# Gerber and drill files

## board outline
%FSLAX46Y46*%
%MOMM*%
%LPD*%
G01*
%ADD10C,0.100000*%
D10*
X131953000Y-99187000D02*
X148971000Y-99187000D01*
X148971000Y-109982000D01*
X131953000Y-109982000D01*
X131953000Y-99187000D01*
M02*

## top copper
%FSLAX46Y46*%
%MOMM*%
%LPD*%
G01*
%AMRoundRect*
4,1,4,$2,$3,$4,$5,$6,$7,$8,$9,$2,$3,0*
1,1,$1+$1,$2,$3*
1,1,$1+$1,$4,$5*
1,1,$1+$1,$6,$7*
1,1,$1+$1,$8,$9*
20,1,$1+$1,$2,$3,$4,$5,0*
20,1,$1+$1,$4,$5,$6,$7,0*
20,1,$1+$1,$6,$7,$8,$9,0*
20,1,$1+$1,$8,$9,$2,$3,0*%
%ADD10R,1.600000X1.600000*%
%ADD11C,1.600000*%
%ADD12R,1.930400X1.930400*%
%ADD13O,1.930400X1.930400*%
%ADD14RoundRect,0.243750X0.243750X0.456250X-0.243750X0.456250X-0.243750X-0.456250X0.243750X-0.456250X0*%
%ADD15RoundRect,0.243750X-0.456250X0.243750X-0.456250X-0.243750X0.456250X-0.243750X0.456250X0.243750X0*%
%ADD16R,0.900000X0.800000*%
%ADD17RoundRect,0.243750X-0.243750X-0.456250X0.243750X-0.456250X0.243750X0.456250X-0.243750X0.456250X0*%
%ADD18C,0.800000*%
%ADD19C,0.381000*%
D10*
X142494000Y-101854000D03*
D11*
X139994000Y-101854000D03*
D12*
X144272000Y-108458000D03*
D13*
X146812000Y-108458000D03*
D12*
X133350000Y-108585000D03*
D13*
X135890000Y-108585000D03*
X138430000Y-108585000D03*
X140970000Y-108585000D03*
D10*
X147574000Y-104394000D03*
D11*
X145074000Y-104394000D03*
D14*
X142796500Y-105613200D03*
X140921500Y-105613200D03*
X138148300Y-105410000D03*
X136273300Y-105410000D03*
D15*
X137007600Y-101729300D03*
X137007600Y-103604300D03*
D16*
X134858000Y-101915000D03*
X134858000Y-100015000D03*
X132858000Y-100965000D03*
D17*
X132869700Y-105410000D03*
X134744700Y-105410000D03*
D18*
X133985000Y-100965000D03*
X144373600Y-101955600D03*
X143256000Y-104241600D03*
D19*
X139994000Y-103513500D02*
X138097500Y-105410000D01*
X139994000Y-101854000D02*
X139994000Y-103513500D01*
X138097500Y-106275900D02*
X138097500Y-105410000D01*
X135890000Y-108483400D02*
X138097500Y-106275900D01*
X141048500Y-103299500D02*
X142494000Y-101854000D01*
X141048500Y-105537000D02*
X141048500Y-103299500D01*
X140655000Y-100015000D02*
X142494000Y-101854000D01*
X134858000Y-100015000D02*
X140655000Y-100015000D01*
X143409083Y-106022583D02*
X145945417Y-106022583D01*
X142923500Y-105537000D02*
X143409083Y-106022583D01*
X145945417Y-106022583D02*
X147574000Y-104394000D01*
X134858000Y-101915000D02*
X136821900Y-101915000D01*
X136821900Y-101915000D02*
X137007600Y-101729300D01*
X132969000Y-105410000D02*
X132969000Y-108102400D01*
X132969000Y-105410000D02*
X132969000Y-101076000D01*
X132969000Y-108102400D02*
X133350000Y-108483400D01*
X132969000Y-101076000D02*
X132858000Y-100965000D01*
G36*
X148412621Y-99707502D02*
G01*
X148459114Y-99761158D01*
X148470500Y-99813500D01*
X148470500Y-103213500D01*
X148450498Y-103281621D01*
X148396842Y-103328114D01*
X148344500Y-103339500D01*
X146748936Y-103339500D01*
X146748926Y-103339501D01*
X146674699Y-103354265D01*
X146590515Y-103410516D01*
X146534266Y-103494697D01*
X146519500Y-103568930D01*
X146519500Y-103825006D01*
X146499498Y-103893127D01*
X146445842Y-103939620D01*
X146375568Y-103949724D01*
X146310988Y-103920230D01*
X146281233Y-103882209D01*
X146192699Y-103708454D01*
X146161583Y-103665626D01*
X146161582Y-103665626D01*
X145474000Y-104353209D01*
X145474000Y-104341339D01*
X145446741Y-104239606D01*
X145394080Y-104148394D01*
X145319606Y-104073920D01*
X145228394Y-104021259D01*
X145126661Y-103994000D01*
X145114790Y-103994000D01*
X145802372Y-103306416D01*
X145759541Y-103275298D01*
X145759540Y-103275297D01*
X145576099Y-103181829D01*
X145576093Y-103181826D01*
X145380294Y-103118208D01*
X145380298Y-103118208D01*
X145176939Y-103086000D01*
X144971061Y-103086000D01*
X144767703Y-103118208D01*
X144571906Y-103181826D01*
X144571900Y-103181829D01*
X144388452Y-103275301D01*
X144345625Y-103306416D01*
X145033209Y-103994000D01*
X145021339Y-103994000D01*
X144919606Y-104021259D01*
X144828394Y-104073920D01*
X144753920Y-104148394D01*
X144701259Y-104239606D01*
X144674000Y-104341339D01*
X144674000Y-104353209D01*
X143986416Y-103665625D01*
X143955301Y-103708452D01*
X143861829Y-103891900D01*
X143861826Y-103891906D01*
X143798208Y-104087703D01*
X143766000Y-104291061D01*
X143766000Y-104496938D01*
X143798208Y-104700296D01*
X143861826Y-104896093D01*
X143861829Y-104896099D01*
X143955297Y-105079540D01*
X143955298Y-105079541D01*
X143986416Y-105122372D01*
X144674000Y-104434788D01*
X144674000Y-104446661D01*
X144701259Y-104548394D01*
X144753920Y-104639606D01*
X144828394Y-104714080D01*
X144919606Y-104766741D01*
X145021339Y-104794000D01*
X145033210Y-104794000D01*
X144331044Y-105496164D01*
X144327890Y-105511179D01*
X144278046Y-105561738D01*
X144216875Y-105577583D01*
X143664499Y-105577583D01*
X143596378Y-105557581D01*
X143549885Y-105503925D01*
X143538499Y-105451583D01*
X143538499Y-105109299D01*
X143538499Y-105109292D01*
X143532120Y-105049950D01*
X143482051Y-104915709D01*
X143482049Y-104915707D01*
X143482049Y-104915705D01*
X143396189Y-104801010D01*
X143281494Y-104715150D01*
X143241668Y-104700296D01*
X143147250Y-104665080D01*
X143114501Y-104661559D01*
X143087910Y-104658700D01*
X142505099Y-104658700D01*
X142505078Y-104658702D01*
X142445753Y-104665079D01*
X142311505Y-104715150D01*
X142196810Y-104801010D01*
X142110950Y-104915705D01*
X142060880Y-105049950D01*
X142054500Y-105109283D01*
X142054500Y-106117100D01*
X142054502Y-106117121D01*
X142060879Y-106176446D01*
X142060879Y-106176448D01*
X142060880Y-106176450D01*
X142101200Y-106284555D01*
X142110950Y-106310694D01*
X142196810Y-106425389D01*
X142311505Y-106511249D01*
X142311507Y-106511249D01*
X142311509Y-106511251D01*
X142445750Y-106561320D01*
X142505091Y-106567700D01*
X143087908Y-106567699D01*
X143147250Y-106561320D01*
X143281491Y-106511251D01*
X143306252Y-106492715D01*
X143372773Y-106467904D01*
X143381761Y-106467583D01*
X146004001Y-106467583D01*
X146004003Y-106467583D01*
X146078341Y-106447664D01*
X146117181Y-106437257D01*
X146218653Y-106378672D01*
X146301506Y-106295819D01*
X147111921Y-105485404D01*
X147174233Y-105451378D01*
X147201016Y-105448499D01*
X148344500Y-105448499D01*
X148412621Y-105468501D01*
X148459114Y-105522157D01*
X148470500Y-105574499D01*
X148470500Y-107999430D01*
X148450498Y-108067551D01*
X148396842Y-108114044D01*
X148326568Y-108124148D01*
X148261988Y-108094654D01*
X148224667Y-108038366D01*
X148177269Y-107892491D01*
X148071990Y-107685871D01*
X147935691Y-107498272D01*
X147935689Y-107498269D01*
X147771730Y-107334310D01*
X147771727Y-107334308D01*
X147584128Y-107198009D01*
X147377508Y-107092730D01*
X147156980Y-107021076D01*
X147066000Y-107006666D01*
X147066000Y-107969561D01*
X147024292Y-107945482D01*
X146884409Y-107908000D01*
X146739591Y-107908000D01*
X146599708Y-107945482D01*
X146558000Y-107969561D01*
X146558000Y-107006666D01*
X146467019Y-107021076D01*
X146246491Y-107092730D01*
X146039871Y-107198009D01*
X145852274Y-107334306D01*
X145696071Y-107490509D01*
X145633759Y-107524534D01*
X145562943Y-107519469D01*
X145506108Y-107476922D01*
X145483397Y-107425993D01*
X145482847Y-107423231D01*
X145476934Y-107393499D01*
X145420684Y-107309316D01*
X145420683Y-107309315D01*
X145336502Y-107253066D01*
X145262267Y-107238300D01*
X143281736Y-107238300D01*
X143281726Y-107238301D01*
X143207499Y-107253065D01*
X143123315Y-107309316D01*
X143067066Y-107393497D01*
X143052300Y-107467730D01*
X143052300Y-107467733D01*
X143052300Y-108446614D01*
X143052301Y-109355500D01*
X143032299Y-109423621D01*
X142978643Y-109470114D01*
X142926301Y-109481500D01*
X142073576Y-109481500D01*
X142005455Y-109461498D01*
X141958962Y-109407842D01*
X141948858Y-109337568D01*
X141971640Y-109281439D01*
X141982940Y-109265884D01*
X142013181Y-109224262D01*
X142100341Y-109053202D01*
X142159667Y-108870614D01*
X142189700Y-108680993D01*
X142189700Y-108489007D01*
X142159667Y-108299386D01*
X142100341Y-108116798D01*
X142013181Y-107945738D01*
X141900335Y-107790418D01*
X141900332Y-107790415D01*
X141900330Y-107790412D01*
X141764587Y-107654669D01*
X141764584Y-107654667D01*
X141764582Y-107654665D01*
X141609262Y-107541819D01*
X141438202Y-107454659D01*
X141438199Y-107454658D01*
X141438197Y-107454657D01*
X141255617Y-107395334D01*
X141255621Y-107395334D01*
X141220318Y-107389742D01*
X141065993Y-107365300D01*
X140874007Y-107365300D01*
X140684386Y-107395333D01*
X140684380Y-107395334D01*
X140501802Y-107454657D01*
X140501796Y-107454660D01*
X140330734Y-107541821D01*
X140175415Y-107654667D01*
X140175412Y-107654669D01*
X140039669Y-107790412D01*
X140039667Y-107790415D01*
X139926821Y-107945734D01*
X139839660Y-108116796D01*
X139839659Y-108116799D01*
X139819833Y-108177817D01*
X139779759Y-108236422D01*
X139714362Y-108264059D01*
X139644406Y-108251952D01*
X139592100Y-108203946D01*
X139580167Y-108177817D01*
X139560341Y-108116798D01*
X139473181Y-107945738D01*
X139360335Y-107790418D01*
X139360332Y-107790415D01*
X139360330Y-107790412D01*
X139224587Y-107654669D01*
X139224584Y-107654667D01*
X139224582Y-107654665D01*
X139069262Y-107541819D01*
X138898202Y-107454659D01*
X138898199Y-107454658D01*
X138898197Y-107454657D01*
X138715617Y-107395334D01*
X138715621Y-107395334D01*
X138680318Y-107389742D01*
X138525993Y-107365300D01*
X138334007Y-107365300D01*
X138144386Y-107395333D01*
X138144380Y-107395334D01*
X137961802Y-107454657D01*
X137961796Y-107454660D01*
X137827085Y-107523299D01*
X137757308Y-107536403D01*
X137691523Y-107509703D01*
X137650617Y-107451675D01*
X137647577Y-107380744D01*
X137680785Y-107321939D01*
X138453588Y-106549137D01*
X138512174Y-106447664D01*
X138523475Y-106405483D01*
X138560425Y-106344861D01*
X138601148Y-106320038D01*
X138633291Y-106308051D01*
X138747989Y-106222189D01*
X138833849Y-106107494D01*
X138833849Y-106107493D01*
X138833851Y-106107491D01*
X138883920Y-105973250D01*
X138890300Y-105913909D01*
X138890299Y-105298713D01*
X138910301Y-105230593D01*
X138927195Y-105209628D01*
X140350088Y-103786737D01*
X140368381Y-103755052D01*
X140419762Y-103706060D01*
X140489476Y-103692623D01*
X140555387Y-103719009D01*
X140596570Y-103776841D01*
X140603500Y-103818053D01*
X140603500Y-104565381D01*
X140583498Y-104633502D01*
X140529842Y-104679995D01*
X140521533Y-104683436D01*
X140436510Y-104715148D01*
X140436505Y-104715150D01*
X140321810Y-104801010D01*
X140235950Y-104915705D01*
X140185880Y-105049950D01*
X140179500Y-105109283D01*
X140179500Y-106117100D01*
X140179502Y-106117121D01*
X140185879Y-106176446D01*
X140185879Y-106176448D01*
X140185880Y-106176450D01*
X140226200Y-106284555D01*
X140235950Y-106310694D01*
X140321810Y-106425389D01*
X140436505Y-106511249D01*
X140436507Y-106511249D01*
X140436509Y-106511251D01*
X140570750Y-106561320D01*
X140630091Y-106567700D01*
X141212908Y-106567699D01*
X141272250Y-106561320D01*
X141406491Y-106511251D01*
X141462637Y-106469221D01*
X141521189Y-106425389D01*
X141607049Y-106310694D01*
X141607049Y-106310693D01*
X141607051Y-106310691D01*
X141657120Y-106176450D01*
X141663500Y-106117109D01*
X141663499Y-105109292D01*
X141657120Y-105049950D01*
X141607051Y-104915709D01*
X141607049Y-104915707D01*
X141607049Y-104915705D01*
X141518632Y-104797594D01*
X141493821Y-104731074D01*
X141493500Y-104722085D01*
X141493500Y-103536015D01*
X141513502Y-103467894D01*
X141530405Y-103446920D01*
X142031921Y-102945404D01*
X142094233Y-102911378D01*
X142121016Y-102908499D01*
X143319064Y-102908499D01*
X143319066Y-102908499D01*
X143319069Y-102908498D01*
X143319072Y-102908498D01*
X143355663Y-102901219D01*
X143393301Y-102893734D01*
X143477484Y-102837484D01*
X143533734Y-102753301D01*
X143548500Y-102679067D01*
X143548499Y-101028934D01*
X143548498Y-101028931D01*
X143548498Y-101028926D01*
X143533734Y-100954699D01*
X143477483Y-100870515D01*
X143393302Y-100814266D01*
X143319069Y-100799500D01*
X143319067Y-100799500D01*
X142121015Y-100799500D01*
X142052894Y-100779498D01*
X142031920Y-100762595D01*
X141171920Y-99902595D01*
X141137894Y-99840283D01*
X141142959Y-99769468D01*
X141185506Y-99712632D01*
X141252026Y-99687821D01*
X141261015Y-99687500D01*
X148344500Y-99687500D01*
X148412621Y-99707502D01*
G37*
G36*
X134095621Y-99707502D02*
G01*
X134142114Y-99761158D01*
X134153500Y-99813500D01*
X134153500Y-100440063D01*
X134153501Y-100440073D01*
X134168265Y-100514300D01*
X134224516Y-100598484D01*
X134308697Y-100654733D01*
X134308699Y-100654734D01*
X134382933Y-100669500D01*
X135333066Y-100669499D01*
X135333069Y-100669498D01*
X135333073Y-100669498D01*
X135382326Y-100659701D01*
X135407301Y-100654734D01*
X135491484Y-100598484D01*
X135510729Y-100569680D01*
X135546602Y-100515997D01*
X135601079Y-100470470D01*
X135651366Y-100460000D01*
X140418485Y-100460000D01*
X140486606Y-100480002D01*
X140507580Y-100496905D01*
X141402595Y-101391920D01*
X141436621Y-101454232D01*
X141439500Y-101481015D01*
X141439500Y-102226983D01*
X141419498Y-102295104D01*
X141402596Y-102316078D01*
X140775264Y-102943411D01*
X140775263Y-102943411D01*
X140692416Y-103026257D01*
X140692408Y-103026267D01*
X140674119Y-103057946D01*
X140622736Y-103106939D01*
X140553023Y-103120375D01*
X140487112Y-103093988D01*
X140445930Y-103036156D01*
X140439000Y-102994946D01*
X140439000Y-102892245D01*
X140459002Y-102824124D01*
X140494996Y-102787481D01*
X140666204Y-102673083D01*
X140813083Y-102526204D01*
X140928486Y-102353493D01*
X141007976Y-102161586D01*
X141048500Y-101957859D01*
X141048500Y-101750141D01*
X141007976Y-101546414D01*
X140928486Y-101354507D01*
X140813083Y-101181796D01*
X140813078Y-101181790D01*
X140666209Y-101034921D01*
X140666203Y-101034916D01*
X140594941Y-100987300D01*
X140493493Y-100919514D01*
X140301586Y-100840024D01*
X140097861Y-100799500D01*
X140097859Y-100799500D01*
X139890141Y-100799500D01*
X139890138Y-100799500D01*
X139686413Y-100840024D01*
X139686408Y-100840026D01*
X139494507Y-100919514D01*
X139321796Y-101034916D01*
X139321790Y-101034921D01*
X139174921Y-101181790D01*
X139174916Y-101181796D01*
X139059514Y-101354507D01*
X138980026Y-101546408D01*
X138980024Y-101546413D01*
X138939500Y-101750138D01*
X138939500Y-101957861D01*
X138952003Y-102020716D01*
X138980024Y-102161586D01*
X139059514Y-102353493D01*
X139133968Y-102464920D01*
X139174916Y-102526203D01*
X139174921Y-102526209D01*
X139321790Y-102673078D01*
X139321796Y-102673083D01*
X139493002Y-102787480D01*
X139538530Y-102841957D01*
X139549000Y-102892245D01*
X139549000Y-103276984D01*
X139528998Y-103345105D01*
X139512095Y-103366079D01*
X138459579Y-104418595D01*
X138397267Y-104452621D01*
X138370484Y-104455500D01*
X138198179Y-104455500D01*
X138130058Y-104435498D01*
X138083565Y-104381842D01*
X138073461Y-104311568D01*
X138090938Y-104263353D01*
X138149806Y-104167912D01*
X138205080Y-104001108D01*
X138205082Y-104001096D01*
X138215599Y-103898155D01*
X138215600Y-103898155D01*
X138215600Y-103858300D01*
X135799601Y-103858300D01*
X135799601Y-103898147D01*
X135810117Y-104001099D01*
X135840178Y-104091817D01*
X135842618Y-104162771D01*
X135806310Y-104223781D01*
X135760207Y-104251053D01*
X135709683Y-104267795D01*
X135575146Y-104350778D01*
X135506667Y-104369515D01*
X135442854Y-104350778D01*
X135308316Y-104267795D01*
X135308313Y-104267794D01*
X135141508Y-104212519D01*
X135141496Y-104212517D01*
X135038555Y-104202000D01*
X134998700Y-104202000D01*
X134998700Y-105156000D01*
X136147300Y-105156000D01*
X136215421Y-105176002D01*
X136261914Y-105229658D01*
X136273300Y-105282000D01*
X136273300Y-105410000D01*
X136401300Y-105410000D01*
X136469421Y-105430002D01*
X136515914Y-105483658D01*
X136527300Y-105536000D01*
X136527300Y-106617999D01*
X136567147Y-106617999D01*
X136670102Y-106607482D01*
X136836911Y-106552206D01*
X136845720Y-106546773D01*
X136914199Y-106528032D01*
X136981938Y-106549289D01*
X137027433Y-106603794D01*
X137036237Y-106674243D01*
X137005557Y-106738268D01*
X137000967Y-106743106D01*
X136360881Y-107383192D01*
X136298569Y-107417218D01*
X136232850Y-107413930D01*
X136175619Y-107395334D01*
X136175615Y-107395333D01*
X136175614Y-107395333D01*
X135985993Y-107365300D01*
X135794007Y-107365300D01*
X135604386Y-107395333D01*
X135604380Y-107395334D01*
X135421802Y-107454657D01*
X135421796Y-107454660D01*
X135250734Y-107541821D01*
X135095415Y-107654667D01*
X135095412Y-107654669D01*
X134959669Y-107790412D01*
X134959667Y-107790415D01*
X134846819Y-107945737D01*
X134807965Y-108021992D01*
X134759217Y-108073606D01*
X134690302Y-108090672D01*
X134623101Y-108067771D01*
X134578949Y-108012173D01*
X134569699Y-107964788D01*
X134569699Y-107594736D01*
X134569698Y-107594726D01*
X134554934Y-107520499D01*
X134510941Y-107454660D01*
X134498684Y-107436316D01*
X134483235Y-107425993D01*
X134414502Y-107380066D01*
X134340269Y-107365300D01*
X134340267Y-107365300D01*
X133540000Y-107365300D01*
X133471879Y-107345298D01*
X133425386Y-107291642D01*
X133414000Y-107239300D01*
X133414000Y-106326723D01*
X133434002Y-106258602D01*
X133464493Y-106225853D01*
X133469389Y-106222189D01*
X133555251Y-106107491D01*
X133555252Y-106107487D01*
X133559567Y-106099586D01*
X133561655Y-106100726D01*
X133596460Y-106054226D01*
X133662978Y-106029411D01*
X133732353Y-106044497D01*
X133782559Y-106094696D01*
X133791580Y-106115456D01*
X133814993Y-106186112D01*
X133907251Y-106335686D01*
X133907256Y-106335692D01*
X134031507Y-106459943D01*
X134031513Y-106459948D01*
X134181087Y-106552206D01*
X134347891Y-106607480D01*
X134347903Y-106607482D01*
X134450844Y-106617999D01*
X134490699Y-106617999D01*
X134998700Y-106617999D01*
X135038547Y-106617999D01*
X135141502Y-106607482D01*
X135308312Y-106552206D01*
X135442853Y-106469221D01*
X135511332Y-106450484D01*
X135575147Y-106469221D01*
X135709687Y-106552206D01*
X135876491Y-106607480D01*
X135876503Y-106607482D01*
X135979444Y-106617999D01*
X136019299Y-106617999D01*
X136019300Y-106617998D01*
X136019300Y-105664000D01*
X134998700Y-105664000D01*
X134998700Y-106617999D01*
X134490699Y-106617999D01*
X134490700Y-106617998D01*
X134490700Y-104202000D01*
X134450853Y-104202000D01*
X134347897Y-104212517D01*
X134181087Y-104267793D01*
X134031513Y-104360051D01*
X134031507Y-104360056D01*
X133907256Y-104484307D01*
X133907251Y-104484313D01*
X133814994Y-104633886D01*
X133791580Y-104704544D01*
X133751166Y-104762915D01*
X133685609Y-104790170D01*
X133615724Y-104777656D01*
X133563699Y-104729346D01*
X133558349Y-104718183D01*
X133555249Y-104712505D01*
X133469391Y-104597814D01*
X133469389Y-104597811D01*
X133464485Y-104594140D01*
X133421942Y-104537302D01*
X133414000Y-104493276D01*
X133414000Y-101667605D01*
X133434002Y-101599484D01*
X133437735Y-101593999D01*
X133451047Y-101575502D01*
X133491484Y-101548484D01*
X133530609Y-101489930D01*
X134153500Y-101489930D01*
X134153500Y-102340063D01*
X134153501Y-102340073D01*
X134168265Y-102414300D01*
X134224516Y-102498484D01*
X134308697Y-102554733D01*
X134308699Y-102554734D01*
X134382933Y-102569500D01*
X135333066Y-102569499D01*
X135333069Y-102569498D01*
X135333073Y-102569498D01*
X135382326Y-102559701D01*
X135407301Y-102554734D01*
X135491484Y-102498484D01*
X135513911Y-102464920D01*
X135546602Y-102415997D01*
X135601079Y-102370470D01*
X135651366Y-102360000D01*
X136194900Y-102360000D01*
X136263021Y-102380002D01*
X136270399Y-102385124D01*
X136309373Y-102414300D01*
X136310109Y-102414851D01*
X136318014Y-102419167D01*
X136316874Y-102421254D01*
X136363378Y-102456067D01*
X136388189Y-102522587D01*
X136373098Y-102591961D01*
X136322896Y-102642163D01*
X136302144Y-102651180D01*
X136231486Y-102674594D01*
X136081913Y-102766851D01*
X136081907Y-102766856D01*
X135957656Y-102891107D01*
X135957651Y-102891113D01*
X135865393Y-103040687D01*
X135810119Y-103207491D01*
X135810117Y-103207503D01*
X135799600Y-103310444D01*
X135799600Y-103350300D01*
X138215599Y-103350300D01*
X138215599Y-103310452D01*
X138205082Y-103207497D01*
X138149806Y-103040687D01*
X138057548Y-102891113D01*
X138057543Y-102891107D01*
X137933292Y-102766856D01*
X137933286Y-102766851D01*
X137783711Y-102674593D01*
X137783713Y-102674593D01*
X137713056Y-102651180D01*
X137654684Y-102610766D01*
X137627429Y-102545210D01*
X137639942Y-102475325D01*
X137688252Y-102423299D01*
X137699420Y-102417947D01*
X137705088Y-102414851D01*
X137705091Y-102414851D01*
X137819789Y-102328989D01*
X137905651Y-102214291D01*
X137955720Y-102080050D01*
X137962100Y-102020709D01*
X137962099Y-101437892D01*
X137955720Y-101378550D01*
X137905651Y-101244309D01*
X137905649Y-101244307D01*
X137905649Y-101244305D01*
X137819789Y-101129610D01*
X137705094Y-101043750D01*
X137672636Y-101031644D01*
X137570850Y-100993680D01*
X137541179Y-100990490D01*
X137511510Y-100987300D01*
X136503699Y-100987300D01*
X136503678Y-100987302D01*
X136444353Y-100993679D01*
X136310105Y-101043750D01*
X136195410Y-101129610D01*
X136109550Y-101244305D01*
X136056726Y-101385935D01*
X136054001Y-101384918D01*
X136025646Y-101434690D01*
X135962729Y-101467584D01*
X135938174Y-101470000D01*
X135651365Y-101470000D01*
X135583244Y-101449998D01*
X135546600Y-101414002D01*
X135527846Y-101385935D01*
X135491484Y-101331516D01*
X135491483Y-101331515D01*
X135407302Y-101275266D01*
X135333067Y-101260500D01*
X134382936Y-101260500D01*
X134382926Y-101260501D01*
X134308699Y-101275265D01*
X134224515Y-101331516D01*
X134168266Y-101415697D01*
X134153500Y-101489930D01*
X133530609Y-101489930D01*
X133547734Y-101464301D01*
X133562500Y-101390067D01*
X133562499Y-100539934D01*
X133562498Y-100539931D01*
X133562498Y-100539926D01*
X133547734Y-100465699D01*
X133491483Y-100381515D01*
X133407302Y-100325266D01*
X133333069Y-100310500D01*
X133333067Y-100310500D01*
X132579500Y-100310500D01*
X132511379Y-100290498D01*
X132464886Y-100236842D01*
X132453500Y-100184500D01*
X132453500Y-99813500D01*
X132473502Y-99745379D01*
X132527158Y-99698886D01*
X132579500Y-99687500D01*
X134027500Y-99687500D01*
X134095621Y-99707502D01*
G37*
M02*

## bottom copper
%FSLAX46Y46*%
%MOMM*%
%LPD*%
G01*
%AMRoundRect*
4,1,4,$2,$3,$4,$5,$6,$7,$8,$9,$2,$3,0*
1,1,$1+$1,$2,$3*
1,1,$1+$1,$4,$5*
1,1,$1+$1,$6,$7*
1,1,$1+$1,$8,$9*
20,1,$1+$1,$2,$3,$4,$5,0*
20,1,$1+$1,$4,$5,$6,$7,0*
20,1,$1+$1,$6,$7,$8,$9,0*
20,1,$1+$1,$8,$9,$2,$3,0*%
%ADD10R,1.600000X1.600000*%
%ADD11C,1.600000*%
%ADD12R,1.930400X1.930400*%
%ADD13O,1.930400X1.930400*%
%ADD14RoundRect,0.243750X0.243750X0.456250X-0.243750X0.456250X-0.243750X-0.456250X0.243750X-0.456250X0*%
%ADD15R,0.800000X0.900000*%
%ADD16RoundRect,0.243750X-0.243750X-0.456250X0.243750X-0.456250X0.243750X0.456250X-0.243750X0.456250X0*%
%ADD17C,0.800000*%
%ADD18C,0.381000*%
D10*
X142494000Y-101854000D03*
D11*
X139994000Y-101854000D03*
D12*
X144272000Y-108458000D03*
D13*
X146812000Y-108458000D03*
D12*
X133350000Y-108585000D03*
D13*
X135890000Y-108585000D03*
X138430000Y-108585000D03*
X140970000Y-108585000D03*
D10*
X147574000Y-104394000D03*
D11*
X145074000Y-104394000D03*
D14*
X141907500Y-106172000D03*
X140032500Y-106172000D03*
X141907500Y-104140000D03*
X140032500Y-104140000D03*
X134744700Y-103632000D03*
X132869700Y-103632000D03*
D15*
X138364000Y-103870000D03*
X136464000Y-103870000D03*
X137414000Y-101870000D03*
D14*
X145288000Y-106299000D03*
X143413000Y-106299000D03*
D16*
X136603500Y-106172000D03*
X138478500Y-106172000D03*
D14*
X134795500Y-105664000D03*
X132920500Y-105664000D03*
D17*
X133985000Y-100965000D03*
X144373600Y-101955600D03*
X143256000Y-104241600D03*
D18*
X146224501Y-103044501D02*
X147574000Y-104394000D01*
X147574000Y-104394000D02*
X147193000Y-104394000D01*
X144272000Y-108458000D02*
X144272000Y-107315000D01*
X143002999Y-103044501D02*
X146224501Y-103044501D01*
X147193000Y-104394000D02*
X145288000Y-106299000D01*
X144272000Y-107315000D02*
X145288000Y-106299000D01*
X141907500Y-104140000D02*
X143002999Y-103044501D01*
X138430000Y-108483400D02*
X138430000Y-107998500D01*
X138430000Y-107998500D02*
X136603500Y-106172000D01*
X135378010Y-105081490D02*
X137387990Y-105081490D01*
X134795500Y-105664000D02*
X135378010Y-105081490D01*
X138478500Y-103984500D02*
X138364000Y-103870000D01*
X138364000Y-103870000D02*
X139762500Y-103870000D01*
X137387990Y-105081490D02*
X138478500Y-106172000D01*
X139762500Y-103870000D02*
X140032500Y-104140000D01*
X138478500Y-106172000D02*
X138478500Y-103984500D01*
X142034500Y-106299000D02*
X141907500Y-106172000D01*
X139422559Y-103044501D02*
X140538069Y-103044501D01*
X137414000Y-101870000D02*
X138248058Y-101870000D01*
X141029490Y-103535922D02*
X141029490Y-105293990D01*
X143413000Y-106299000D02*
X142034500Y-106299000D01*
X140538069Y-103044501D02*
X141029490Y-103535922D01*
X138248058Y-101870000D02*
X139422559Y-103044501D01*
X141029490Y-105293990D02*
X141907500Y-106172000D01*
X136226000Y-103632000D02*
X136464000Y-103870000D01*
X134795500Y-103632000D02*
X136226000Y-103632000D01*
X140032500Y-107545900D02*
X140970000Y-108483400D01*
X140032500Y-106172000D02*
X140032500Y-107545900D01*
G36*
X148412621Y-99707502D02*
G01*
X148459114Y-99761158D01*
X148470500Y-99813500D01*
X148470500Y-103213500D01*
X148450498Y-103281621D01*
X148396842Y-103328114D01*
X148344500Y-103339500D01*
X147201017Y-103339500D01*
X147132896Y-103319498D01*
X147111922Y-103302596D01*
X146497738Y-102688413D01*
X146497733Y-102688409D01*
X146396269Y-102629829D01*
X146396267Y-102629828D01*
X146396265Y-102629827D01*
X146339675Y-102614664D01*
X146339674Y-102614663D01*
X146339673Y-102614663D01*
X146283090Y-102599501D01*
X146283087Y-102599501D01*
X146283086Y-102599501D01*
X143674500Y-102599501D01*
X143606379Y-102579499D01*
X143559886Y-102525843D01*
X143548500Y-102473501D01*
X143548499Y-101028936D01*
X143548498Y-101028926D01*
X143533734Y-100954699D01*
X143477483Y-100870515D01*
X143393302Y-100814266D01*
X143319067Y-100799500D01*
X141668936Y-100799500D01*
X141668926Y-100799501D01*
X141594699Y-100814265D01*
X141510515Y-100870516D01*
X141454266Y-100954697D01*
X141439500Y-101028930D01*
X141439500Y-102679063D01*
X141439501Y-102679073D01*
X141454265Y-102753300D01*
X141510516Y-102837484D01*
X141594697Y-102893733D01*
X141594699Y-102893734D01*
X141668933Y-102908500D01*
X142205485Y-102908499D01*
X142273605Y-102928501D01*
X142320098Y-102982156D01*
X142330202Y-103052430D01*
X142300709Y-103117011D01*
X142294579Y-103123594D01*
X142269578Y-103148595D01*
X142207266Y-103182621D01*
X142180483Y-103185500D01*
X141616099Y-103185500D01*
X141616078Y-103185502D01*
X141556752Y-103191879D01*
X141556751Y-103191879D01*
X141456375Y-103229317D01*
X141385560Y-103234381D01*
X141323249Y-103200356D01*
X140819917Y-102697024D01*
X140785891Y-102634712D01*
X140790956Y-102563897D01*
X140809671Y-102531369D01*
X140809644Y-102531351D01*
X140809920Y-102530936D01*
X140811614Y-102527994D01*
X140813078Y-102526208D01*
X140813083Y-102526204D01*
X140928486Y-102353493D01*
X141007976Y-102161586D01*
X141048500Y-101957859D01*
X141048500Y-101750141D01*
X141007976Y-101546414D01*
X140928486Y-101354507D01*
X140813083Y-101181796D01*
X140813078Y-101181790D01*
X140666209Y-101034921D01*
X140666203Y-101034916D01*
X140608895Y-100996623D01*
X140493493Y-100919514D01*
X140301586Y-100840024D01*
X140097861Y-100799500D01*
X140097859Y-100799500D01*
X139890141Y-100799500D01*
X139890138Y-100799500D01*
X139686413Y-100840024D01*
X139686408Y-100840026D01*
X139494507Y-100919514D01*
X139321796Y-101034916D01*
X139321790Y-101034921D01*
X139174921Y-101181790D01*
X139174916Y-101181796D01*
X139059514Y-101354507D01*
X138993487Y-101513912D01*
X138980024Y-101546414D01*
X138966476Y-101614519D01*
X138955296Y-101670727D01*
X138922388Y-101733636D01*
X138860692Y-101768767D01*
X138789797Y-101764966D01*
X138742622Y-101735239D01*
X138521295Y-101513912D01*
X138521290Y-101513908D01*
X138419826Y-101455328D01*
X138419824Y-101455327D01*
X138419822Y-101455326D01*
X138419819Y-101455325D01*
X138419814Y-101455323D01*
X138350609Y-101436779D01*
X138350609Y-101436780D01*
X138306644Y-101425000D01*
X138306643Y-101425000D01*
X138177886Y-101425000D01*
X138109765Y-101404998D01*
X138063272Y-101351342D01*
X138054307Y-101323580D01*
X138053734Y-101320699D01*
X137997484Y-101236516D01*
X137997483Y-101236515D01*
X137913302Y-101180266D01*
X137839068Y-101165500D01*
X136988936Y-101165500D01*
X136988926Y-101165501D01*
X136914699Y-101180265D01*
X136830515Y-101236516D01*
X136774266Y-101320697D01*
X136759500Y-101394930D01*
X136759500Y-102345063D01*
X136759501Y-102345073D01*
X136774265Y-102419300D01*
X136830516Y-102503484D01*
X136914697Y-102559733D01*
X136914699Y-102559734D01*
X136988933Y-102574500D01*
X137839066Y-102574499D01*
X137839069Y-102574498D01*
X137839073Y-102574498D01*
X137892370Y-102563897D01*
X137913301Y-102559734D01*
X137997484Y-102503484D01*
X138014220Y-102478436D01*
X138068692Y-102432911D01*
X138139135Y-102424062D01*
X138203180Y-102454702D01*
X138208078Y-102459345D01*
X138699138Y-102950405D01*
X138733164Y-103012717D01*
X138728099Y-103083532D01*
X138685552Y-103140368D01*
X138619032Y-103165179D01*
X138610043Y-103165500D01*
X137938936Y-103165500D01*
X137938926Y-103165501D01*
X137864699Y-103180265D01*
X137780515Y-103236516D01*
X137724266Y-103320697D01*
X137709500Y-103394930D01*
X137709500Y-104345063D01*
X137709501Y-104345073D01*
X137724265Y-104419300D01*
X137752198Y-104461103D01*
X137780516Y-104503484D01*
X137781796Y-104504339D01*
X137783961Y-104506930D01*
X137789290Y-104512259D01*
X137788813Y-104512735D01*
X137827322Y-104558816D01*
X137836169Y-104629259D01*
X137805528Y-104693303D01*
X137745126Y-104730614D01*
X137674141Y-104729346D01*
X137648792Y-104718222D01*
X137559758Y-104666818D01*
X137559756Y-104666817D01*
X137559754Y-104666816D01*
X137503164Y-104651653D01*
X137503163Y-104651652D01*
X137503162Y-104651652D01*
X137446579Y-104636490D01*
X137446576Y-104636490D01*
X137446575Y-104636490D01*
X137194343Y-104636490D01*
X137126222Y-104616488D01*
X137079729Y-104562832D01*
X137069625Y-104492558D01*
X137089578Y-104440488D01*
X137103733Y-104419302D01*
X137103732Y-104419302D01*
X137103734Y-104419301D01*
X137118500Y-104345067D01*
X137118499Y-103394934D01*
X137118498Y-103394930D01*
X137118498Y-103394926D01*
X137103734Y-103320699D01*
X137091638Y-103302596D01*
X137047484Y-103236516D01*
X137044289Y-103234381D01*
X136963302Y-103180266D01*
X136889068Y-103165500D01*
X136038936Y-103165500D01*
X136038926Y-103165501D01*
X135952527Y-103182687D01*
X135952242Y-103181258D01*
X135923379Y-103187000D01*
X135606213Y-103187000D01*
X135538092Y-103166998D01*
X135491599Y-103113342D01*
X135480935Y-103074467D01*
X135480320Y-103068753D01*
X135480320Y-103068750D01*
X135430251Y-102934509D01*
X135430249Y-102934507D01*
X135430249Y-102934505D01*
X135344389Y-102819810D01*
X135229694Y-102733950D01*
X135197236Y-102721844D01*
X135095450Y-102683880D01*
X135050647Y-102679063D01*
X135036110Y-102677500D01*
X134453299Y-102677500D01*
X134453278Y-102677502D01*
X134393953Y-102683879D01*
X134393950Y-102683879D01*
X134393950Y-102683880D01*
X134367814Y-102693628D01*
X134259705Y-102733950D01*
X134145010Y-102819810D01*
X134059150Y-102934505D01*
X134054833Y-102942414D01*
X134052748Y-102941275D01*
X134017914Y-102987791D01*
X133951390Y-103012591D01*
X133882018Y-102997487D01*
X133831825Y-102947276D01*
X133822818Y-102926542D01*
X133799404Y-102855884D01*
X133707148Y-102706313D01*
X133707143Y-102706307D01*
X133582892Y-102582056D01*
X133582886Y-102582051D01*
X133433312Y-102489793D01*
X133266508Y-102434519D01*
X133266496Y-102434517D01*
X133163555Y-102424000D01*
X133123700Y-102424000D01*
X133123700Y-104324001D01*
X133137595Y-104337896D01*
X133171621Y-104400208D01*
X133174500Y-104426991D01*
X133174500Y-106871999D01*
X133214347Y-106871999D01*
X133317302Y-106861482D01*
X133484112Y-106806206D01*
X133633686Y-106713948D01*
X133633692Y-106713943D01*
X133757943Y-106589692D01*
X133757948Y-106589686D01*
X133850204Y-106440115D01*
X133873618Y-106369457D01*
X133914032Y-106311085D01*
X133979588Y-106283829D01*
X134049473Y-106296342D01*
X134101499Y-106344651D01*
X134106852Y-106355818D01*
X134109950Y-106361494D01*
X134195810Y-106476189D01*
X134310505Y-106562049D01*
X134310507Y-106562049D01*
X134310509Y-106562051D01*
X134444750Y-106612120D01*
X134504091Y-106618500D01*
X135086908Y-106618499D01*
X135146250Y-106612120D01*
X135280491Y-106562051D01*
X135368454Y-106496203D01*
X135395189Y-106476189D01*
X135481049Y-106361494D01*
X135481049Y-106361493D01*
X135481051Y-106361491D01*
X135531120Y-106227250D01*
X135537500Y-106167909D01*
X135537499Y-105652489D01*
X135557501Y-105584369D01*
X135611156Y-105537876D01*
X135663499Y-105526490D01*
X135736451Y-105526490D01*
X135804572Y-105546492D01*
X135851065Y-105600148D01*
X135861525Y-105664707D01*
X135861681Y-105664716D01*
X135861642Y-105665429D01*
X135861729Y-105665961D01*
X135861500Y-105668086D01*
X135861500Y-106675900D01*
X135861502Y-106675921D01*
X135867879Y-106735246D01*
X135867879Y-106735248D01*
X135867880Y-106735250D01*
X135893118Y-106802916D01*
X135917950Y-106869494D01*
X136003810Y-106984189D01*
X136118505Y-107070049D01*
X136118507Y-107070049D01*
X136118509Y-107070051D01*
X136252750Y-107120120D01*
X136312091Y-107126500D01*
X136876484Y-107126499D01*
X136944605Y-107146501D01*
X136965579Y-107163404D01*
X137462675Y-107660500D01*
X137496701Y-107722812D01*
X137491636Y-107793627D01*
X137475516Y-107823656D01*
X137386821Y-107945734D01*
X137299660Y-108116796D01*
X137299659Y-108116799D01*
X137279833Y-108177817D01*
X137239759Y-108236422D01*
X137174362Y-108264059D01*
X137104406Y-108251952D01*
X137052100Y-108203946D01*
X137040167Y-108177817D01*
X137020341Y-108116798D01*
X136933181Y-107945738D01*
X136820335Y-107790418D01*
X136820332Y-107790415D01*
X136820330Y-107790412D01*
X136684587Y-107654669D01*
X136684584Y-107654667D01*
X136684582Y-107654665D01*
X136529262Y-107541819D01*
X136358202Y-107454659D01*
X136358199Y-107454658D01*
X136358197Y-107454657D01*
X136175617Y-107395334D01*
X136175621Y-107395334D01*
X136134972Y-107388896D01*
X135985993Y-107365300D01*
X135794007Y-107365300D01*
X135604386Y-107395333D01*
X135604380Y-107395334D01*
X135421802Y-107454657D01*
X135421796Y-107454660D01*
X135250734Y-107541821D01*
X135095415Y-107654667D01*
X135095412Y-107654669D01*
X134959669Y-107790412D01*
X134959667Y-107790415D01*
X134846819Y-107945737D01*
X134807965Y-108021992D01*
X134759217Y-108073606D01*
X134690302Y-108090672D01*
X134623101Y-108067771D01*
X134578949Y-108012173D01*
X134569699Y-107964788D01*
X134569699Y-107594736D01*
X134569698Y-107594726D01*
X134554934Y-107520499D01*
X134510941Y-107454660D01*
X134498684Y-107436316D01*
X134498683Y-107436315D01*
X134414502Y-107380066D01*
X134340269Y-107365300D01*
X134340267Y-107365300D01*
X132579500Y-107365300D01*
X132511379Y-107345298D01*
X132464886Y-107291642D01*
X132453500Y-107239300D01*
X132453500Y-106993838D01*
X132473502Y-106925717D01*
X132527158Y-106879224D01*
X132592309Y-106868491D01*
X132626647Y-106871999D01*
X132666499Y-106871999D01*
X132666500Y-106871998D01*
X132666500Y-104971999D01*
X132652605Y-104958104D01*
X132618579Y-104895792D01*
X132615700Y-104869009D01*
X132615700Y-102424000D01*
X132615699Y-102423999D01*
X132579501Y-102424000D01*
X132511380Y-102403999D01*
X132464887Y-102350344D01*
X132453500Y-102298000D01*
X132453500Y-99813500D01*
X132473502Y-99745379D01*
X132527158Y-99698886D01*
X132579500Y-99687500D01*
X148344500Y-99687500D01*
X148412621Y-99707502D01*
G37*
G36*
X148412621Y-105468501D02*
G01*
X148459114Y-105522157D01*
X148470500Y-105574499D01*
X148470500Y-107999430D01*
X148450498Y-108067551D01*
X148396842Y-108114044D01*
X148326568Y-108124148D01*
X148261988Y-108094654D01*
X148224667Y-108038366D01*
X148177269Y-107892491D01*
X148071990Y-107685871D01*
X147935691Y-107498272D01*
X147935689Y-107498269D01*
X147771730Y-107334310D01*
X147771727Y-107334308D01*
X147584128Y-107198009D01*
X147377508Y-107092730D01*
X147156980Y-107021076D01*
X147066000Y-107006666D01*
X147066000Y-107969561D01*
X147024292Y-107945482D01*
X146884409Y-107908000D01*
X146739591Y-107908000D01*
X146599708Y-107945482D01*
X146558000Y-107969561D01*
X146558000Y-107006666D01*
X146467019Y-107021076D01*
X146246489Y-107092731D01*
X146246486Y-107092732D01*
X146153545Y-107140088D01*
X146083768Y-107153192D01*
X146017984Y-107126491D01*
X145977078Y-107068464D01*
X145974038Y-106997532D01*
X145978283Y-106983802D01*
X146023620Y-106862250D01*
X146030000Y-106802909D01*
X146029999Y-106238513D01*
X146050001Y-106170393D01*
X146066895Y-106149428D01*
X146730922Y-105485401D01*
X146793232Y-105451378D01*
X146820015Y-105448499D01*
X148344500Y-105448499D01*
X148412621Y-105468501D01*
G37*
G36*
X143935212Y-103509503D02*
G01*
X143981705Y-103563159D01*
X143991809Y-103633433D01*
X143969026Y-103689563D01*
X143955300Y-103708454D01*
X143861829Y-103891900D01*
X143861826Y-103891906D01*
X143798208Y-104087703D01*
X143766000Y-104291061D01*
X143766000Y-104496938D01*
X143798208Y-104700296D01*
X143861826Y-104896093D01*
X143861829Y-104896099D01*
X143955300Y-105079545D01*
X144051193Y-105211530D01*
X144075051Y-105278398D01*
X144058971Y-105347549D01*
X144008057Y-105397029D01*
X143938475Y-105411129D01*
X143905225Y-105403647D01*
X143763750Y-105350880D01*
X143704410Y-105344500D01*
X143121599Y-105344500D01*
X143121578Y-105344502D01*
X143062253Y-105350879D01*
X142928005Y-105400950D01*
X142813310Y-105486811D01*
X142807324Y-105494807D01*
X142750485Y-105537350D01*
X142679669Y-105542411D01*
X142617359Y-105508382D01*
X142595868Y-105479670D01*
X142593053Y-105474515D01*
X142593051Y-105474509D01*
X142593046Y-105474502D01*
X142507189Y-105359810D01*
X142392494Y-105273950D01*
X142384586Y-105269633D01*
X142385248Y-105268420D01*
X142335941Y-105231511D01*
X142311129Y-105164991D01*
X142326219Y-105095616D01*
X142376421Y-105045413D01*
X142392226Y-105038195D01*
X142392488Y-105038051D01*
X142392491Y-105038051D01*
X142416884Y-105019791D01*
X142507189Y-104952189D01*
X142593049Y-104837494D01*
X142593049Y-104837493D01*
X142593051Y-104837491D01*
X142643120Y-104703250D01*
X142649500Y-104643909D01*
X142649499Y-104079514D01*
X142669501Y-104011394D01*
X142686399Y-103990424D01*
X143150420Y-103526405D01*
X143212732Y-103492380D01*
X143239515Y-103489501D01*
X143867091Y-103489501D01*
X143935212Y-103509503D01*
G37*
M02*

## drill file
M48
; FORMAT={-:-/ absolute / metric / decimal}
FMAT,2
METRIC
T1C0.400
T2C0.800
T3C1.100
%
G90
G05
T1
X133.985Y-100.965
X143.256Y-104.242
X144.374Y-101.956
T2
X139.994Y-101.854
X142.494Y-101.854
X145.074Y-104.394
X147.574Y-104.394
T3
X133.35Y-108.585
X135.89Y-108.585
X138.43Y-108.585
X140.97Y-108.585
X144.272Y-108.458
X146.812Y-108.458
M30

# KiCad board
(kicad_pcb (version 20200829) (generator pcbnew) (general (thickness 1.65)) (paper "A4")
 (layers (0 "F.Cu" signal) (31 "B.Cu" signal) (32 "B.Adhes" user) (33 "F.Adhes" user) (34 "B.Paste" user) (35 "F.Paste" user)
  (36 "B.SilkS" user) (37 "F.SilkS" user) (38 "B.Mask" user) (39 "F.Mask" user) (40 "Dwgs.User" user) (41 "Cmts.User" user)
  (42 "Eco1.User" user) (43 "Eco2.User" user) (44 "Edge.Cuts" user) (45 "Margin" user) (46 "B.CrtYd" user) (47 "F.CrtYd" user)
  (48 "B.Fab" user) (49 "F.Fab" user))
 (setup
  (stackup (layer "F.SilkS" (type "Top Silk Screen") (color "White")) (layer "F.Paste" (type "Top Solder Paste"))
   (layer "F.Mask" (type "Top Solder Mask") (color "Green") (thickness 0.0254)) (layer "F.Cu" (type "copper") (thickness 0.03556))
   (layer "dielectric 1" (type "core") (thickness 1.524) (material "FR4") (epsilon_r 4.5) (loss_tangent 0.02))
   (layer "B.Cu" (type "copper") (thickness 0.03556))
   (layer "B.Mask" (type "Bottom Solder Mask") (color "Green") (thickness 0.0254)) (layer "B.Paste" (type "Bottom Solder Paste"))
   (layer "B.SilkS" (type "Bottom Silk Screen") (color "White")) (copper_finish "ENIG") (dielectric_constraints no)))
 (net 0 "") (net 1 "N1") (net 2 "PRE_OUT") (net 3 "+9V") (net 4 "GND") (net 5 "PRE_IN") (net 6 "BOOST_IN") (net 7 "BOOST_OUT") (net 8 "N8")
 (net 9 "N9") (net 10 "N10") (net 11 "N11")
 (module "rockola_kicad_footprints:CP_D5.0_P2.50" (layer "F.Cu") (at 142.494 101.854 180)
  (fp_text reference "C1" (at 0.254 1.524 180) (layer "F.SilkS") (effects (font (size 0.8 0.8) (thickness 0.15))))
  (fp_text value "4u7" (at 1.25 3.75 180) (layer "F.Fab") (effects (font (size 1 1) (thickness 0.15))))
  (pad "1" thru_hole rect (at 0 0 180) (size 1.6 1.6) (drill 0.8) (layers *.Cu *.Mask) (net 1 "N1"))
  (pad "2" thru_hole circle (at 2.5 0 180) (size 1.6 1.6) (drill 0.8) (layers *.Cu *.Mask) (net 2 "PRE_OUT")))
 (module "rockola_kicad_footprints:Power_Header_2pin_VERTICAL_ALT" (layer "F.Cu") (at 145.542 109.728 -90)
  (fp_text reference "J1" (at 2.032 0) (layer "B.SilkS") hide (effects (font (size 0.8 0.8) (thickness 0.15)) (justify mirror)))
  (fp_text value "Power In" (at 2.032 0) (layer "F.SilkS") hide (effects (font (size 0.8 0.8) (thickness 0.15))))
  (pad "1" thru_hole rect (at -1.27 1.27) (size 1.9304 1.9304) (drill 1.1) (layers *.Cu *.Mask) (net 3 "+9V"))
  (pad "2" thru_hole oval (at -1.27 -1.27) (size 1.9304 1.9304) (drill 1.1) (layers *.Cu *.Mask) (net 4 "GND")))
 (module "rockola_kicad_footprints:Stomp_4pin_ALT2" (layer "F.Cu") (at 137.16 108.585)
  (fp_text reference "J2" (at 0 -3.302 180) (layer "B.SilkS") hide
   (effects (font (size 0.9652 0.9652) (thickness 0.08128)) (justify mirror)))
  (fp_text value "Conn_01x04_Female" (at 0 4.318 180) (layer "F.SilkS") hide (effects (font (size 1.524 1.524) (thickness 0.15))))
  (pad "1" thru_hole rect (at -3.81 0) (size 1.9304 1.9304) (drill 1.1) (layers *.Cu *.Mask) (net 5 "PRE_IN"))
  (pad "2" thru_hole oval (at -1.27 0) (size 1.9304 1.9304) (drill 1.1) (layers *.Cu *.Mask) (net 2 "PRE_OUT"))
  (pad "3" thru_hole oval (at 1.27 0) (size 1.9304 1.9304) (drill 1.1) (layers *.Cu *.Mask) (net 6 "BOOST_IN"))
  (pad "4" thru_hole oval (at 3.81 0) (size 1.9304 1.9304) (drill 1.1) (layers *.Cu *.Mask) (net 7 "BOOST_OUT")))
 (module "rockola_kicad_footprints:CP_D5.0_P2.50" (layer "F.Cu") (at 147.574 104.394 180)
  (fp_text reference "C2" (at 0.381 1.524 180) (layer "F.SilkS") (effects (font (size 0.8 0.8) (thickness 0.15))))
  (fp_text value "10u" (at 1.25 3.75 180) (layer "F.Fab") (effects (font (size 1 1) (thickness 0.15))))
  (pad "1" thru_hole rect (at 0 0 180) (size 1.6 1.6) (drill 0.8) (layers *.Cu *.Mask) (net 3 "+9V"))
  (pad "2" thru_hole circle (at 2.5 0 180) (size 1.6 1.6) (drill 0.8) (layers *.Cu *.Mask) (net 4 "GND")))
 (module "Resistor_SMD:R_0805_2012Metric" (layer "F.Cu") (at 141.859 105.6132 180)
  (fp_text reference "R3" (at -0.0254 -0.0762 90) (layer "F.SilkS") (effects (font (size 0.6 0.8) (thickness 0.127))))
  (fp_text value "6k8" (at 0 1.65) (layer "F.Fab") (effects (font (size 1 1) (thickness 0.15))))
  (pad "1" smd roundrect (at -0.9375 0 180) (size 0.975 1.4) (layers "F.Cu" "F.Paste" "F.Mask") (roundrect_rratio 0.25) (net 3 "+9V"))
  (pad "2" smd roundrect (at 0.9375 0 180) (size 0.975 1.4) (layers "F.Cu" "F.Paste" "F.Mask") (roundrect_rratio 0.25) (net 1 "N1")))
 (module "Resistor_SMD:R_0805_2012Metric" (layer "F.Cu") (at 137.2108 105.41 180)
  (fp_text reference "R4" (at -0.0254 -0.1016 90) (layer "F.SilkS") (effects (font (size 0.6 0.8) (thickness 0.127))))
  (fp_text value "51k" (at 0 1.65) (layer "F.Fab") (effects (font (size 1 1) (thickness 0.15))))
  (pad "1" smd roundrect (at -0.9375 0 180) (size 0.975 1.4) (layers "F.Cu" "F.Paste" "F.Mask") (roundrect_rratio 0.25) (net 2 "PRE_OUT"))
  (pad "2" smd roundrect (at 0.9375 0 180) (size 0.975 1.4) (layers "F.Cu" "F.Paste" "F.Mask") (roundrect_rratio 0.25) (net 4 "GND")))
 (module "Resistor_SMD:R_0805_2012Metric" (layer "F.Cu") (at 137.0076 102.6668 -90)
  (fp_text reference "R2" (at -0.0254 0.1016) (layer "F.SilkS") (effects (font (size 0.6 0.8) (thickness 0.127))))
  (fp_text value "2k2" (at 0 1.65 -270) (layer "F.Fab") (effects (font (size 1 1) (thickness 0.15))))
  (pad "1" smd roundrect (at -0.9375 0 270) (size 0.975 1.4) (layers "F.Cu" "F.Paste" "F.Mask") (roundrect_rratio 0.25) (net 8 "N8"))
  (pad "2" smd roundrect (at 0.9375 0 270) (size 0.975 1.4) (layers "F.Cu" "F.Paste" "F.Mask") (roundrect_rratio 0.25) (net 4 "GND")))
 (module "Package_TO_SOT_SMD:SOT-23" (layer "F.Cu") (at 133.858 100.965 180)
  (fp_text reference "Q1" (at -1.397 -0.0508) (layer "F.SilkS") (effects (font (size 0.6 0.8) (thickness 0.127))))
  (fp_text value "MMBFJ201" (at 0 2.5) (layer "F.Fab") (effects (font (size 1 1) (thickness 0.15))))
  (pad "1" smd rect (at -1 -0.95 180) (size 0.9 0.8) (layers "F.Cu" "F.Paste" "F.Mask") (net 8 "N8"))
  (pad "2" smd rect (at -1 0.95 180) (size 0.9 0.8) (layers "F.Cu" "F.Paste" "F.Mask") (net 1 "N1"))
  (pad "3" smd rect (at 1 0 180) (size 0.9 0.8) (layers "F.Cu" "F.Paste" "F.Mask") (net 5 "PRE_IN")))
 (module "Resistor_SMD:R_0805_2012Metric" (layer "F.Cu") (at 133.8072 105.41)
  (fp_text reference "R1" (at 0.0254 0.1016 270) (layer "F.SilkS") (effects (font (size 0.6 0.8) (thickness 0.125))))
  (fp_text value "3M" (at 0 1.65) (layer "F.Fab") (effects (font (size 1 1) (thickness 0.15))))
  (pad "1" smd roundrect (at -0.9375 0) (size 0.975 1.4) (layers "F.Cu" "F.Paste" "F.Mask") (roundrect_rratio 0.25) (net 5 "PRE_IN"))
  (pad "2" smd roundrect (at 0.9375 0) (size 0.975 1.4) (layers "F.Cu" "F.Paste" "F.Mask") (roundrect_rratio 0.25) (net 4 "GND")))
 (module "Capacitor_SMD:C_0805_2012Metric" (layer "B.Cu") (at 140.97 106.172 180)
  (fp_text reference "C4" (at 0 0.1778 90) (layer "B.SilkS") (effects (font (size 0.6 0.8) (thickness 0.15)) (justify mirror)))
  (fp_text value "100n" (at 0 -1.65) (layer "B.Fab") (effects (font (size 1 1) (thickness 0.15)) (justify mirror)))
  (pad "1" smd roundrect (at -0.9375 0 180) (size 0.975 1.4) (layers "B.Cu" "B.Paste" "B.Mask") (roundrect_rratio 0.25) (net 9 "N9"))
  (pad "2" smd roundrect (at 0.9375 0 180) (size 0.975 1.4) (layers "B.Cu" "B.Paste" "B.Mask") (roundrect_rratio 0.25) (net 7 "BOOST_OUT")))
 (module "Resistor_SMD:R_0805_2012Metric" (layer "B.Cu") (at 140.97 104.14 180)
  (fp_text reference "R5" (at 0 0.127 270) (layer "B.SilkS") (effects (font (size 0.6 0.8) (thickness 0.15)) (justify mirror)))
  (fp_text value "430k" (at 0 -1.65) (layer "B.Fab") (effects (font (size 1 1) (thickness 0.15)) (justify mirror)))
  (pad "1" smd roundrect (at -0.9375 0 180) (size 0.975 1.4) (layers "B.Cu" "B.Paste" "B.Mask") (roundrect_rratio 0.25) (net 3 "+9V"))
  (pad "2" smd roundrect (at 0.9375 0 180) (size 0.975 1.4) (layers "B.Cu" "B.Paste" "B.Mask") (roundrect_rratio 0.25) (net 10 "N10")))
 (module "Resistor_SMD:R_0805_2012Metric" (layer "B.Cu") (at 133.8072 103.632 180)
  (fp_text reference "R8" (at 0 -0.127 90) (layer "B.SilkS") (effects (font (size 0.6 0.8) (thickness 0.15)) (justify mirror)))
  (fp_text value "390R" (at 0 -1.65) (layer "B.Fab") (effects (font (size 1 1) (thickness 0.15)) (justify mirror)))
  (pad "1" smd roundrect (at -0.9375 0 180) (size 0.975 1.4) (layers "B.Cu" "B.Paste" "B.Mask") (roundrect_rratio 0.25) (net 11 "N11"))
  (pad "2" smd roundrect (at 0.9375 0 180) (size 0.975 1.4) (layers "B.Cu" "B.Paste" "B.Mask") (roundrect_rratio 0.25) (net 4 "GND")))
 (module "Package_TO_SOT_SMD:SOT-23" (layer "B.Cu") (at 137.414 102.87 90)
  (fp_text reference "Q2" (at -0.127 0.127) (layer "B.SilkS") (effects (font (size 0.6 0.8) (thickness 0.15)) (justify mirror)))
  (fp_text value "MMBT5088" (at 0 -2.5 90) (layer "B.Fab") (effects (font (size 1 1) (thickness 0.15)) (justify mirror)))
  (pad "1" smd rect (at -1 0.95 90) (size 0.9 0.8) (layers "B.Cu" "B.Paste" "B.Mask") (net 10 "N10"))
  (pad "2" smd rect (at -1 -0.95 90) (size 0.9 0.8) (layers "B.Cu" "B.Paste" "B.Mask") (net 11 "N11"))
  (pad "3" smd rect (at 1 0 90) (size 0.9 0.8) (layers "B.Cu" "B.Paste" "B.Mask") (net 9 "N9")))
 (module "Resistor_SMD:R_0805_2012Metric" (layer "B.Cu") (at 144.3505 106.299 180)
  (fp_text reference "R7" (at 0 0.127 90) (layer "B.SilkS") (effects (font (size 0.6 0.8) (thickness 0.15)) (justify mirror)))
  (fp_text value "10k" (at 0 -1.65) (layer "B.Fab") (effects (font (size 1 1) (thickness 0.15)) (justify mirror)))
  (pad "1" smd roundrect (at -0.9375 0 180) (size 0.975 1.4) (layers "B.Cu" "B.Paste" "B.Mask") (roundrect_rratio 0.25) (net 3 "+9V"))
  (pad "2" smd roundrect (at 0.9375 0 180) (size 0.975 1.4) (layers "B.Cu" "B.Paste" "B.Mask") (roundrect_rratio 0.25) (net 9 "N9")))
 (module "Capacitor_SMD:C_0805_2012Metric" (layer "B.Cu") (at 137.541 106.172)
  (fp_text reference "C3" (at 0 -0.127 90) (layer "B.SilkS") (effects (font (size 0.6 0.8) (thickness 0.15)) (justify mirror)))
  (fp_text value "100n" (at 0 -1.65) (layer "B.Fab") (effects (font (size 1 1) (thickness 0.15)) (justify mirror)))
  (pad "1" smd roundrect (at -0.9375 0) (size 0.975 1.4) (layers "B.Cu" "B.Paste" "B.Mask") (roundrect_rratio 0.25) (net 6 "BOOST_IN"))
  (pad "2" smd roundrect (at 0.9375 0) (size 0.975 1.4) (layers "B.Cu" "B.Paste" "B.Mask") (roundrect_rratio 0.25) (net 10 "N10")))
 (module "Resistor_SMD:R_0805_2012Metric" (layer "B.Cu") (at 133.858 105.664 180)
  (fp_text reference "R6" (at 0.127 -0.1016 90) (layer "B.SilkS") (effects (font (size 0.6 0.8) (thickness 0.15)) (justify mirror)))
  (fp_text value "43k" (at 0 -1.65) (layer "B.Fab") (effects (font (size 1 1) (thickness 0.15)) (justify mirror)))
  (pad "1" smd roundrect (at -0.9375 0 180) (size 0.975 1.4) (layers "B.Cu" "B.Paste" "B.Mask") (roundrect_rratio 0.25) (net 10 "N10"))
  (pad "2" smd roundrect (at 0.9375 0 180) (size 0.975 1.4) (layers "B.Cu" "B.Paste" "B.Mask") (roundrect_rratio 0.25) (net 4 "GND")))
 (gr_rect (start 131.953 99.187) (end 148.971 109.982) (layer "Edge.Cuts") (width 0.1))
 (segment (start 139.994 103.5135) (end 138.0975 105.41) (width 0.381) (layer "F.Cu") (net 2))
 (segment (start 139.994 101.854) (end 139.994 103.5135) (width 0.381) (layer "F.Cu") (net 2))
 (segment (start 138.0975 106.2759) (end 138.0975 105.41) (width 0.381) (layer "F.Cu") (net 2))
 (segment (start 135.89 108.4834) (end 138.0975 106.2759) (width 0.381) (layer "F.Cu") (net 2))
 (segment (start 141.0485 103.2995) (end 142.494 101.854) (width 0.381) (layer "F.Cu") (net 1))
 (segment (start 141.0485 105.537) (end 141.0485 103.2995) (width 0.381) (layer "F.Cu") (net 1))
 (segment (start 140.655 100.015) (end 142.494 101.854) (width 0.381) (layer "F.Cu") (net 1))
 (segment (start 134.858 100.015) (end 140.655 100.015) (width 0.381) (layer "F.Cu") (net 1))
 (via (at 133.985 100.965) (size 0.8) (drill 0.4) (layers "F.Cu" "B.Cu") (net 4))
 (via (at 144.3736 101.9556) (size 0.8) (drill 0.4) (layers "F.Cu" "B.Cu") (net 4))
 (via (at 143.256 104.2416) (size 0.8) (drill 0.4) (layers "F.Cu" "B.Cu") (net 4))
 (segment (start 143.409083 106.022583) (end 145.945417 106.022583) (width 0.381) (layer "F.Cu") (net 3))
 (segment (start 142.9235 105.537) (end 143.409083 106.022583) (width 0.381) (layer "F.Cu") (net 3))
 (segment (start 145.945417 106.022583) (end 147.574 104.394) (width 0.381) (layer "F.Cu") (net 3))
 (segment (start 146.224501 103.044501) (end 147.574 104.394) (width 0.381) (layer "B.Cu") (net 3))
 (segment (start 147.574 104.394) (end 147.193 104.394) (width 0.381) (layer "B.Cu") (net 3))
 (segment (start 144.272 108.458) (end 144.272 107.315) (width 0.381) (layer "B.Cu") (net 3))
 (segment (start 143.002999 103.044501) (end 146.224501 103.044501) (width 0.381) (layer "B.Cu") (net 3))
 (segment (start 147.193 104.394) (end 145.288 106.299) (width 0.381) (layer "B.Cu") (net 3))
 (segment (start 144.272 107.315) (end 145.288 106.299) (width 0.381) (layer "B.Cu") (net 3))
 (segment (start 141.9075 104.14) (end 143.002999 103.044501) (width 0.381) (layer "B.Cu") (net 3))
 (segment (start 138.43 108.4834) (end 138.43 107.9985) (width 0.381) (layer "B.Cu") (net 6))
 (segment (start 138.43 107.9985) (end 136.6035 106.172) (width 0.381) (layer "B.Cu") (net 6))
 (segment (start 134.858 101.915) (end 136.8219 101.915) (width 0.381) (layer "F.Cu") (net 8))
 (segment (start 136.8219 101.915) (end 137.0076 101.7293) (width 0.381) (layer "F.Cu") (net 8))
 (segment (start 135.37801 105.08149) (end 137.38799 105.08149) (width 0.381) (layer "B.Cu") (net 10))
 (segment (start 134.7955 105.664) (end 135.37801 105.08149) (width 0.381) (layer "B.Cu") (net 10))
 (segment (start 138.4785 103.9845) (end 138.364 103.87) (width 0.381) (layer "B.Cu") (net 10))
 (segment (start 138.364 103.87) (end 139.7625 103.87) (width 0.381) (layer "B.Cu") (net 10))
 (segment (start 137.38799 105.08149) (end 138.4785 106.172) (width 0.381) (layer "B.Cu") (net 10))
 (segment (start 139.7625 103.87) (end 140.0325 104.14) (width 0.381) (layer "B.Cu") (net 10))
 (segment (start 138.4785 106.172) (end 138.4785 103.9845) (width 0.381) (layer "B.Cu") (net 10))
 (segment (start 142.0345 106.299) (end 141.9075 106.172) (width 0.381) (layer "B.Cu") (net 9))
 (segment (start 139.422559 103.044501) (end 140.538069 103.044501) (width 0.381) (layer "B.Cu") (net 9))
 (segment (start 137.414 101.87) (end 138.248058 101.87) (width 0.381) (layer "B.Cu") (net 9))
 (segment (start 141.02949 103.535922) (end 141.02949 105.29399) (width 0.381) (layer "B.Cu") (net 9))
 (segment (start 143.413 106.299) (end 142.0345 106.299) (width 0.381) (layer "B.Cu") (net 9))
 (segment (start 140.538069 103.044501) (end 141.02949 103.535922) (width 0.381) (layer "B.Cu") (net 9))
 (segment (start 138.248058 101.87) (end 139.422559 103.044501) (width 0.381) (layer "B.Cu") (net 9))
 (segment (start 141.02949 105.29399) (end 141.9075 106.172) (width 0.381) (layer "B.Cu") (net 9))
 (segment (start 136.226 103.632) (end 136.464 103.87) (width 0.381) (layer "B.Cu") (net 11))
 (segment (start 134.7955 103.632) (end 136.226 103.632) (width 0.381) (layer "B.Cu") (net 11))
 (segment (start 140.0325 107.5459) (end 140.97 108.4834) (width 0.381) (layer "B.Cu") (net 7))
 (segment (start 140.0325 106.172) (end 140.0325 107.5459) (width 0.381) (layer "B.Cu") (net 7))
 (segment (start 132.969 105.41) (end 132.969 108.1024) (width 0.381) (layer "F.Cu") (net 5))
 (segment (start 132.969 105.41) (end 132.969 101.076) (width 0.381) (layer "F.Cu") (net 5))
 (segment (start 132.969 108.1024) (end 133.35 108.4834) (width 0.381) (layer "F.Cu") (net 5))
 (segment (start 132.969 101.076) (end 132.858 100.965) (width 0.381) (layer "F.Cu") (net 5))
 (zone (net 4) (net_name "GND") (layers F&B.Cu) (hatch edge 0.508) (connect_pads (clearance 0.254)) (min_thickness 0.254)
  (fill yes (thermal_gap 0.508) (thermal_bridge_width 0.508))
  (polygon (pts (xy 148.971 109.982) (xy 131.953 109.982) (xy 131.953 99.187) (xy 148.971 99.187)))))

